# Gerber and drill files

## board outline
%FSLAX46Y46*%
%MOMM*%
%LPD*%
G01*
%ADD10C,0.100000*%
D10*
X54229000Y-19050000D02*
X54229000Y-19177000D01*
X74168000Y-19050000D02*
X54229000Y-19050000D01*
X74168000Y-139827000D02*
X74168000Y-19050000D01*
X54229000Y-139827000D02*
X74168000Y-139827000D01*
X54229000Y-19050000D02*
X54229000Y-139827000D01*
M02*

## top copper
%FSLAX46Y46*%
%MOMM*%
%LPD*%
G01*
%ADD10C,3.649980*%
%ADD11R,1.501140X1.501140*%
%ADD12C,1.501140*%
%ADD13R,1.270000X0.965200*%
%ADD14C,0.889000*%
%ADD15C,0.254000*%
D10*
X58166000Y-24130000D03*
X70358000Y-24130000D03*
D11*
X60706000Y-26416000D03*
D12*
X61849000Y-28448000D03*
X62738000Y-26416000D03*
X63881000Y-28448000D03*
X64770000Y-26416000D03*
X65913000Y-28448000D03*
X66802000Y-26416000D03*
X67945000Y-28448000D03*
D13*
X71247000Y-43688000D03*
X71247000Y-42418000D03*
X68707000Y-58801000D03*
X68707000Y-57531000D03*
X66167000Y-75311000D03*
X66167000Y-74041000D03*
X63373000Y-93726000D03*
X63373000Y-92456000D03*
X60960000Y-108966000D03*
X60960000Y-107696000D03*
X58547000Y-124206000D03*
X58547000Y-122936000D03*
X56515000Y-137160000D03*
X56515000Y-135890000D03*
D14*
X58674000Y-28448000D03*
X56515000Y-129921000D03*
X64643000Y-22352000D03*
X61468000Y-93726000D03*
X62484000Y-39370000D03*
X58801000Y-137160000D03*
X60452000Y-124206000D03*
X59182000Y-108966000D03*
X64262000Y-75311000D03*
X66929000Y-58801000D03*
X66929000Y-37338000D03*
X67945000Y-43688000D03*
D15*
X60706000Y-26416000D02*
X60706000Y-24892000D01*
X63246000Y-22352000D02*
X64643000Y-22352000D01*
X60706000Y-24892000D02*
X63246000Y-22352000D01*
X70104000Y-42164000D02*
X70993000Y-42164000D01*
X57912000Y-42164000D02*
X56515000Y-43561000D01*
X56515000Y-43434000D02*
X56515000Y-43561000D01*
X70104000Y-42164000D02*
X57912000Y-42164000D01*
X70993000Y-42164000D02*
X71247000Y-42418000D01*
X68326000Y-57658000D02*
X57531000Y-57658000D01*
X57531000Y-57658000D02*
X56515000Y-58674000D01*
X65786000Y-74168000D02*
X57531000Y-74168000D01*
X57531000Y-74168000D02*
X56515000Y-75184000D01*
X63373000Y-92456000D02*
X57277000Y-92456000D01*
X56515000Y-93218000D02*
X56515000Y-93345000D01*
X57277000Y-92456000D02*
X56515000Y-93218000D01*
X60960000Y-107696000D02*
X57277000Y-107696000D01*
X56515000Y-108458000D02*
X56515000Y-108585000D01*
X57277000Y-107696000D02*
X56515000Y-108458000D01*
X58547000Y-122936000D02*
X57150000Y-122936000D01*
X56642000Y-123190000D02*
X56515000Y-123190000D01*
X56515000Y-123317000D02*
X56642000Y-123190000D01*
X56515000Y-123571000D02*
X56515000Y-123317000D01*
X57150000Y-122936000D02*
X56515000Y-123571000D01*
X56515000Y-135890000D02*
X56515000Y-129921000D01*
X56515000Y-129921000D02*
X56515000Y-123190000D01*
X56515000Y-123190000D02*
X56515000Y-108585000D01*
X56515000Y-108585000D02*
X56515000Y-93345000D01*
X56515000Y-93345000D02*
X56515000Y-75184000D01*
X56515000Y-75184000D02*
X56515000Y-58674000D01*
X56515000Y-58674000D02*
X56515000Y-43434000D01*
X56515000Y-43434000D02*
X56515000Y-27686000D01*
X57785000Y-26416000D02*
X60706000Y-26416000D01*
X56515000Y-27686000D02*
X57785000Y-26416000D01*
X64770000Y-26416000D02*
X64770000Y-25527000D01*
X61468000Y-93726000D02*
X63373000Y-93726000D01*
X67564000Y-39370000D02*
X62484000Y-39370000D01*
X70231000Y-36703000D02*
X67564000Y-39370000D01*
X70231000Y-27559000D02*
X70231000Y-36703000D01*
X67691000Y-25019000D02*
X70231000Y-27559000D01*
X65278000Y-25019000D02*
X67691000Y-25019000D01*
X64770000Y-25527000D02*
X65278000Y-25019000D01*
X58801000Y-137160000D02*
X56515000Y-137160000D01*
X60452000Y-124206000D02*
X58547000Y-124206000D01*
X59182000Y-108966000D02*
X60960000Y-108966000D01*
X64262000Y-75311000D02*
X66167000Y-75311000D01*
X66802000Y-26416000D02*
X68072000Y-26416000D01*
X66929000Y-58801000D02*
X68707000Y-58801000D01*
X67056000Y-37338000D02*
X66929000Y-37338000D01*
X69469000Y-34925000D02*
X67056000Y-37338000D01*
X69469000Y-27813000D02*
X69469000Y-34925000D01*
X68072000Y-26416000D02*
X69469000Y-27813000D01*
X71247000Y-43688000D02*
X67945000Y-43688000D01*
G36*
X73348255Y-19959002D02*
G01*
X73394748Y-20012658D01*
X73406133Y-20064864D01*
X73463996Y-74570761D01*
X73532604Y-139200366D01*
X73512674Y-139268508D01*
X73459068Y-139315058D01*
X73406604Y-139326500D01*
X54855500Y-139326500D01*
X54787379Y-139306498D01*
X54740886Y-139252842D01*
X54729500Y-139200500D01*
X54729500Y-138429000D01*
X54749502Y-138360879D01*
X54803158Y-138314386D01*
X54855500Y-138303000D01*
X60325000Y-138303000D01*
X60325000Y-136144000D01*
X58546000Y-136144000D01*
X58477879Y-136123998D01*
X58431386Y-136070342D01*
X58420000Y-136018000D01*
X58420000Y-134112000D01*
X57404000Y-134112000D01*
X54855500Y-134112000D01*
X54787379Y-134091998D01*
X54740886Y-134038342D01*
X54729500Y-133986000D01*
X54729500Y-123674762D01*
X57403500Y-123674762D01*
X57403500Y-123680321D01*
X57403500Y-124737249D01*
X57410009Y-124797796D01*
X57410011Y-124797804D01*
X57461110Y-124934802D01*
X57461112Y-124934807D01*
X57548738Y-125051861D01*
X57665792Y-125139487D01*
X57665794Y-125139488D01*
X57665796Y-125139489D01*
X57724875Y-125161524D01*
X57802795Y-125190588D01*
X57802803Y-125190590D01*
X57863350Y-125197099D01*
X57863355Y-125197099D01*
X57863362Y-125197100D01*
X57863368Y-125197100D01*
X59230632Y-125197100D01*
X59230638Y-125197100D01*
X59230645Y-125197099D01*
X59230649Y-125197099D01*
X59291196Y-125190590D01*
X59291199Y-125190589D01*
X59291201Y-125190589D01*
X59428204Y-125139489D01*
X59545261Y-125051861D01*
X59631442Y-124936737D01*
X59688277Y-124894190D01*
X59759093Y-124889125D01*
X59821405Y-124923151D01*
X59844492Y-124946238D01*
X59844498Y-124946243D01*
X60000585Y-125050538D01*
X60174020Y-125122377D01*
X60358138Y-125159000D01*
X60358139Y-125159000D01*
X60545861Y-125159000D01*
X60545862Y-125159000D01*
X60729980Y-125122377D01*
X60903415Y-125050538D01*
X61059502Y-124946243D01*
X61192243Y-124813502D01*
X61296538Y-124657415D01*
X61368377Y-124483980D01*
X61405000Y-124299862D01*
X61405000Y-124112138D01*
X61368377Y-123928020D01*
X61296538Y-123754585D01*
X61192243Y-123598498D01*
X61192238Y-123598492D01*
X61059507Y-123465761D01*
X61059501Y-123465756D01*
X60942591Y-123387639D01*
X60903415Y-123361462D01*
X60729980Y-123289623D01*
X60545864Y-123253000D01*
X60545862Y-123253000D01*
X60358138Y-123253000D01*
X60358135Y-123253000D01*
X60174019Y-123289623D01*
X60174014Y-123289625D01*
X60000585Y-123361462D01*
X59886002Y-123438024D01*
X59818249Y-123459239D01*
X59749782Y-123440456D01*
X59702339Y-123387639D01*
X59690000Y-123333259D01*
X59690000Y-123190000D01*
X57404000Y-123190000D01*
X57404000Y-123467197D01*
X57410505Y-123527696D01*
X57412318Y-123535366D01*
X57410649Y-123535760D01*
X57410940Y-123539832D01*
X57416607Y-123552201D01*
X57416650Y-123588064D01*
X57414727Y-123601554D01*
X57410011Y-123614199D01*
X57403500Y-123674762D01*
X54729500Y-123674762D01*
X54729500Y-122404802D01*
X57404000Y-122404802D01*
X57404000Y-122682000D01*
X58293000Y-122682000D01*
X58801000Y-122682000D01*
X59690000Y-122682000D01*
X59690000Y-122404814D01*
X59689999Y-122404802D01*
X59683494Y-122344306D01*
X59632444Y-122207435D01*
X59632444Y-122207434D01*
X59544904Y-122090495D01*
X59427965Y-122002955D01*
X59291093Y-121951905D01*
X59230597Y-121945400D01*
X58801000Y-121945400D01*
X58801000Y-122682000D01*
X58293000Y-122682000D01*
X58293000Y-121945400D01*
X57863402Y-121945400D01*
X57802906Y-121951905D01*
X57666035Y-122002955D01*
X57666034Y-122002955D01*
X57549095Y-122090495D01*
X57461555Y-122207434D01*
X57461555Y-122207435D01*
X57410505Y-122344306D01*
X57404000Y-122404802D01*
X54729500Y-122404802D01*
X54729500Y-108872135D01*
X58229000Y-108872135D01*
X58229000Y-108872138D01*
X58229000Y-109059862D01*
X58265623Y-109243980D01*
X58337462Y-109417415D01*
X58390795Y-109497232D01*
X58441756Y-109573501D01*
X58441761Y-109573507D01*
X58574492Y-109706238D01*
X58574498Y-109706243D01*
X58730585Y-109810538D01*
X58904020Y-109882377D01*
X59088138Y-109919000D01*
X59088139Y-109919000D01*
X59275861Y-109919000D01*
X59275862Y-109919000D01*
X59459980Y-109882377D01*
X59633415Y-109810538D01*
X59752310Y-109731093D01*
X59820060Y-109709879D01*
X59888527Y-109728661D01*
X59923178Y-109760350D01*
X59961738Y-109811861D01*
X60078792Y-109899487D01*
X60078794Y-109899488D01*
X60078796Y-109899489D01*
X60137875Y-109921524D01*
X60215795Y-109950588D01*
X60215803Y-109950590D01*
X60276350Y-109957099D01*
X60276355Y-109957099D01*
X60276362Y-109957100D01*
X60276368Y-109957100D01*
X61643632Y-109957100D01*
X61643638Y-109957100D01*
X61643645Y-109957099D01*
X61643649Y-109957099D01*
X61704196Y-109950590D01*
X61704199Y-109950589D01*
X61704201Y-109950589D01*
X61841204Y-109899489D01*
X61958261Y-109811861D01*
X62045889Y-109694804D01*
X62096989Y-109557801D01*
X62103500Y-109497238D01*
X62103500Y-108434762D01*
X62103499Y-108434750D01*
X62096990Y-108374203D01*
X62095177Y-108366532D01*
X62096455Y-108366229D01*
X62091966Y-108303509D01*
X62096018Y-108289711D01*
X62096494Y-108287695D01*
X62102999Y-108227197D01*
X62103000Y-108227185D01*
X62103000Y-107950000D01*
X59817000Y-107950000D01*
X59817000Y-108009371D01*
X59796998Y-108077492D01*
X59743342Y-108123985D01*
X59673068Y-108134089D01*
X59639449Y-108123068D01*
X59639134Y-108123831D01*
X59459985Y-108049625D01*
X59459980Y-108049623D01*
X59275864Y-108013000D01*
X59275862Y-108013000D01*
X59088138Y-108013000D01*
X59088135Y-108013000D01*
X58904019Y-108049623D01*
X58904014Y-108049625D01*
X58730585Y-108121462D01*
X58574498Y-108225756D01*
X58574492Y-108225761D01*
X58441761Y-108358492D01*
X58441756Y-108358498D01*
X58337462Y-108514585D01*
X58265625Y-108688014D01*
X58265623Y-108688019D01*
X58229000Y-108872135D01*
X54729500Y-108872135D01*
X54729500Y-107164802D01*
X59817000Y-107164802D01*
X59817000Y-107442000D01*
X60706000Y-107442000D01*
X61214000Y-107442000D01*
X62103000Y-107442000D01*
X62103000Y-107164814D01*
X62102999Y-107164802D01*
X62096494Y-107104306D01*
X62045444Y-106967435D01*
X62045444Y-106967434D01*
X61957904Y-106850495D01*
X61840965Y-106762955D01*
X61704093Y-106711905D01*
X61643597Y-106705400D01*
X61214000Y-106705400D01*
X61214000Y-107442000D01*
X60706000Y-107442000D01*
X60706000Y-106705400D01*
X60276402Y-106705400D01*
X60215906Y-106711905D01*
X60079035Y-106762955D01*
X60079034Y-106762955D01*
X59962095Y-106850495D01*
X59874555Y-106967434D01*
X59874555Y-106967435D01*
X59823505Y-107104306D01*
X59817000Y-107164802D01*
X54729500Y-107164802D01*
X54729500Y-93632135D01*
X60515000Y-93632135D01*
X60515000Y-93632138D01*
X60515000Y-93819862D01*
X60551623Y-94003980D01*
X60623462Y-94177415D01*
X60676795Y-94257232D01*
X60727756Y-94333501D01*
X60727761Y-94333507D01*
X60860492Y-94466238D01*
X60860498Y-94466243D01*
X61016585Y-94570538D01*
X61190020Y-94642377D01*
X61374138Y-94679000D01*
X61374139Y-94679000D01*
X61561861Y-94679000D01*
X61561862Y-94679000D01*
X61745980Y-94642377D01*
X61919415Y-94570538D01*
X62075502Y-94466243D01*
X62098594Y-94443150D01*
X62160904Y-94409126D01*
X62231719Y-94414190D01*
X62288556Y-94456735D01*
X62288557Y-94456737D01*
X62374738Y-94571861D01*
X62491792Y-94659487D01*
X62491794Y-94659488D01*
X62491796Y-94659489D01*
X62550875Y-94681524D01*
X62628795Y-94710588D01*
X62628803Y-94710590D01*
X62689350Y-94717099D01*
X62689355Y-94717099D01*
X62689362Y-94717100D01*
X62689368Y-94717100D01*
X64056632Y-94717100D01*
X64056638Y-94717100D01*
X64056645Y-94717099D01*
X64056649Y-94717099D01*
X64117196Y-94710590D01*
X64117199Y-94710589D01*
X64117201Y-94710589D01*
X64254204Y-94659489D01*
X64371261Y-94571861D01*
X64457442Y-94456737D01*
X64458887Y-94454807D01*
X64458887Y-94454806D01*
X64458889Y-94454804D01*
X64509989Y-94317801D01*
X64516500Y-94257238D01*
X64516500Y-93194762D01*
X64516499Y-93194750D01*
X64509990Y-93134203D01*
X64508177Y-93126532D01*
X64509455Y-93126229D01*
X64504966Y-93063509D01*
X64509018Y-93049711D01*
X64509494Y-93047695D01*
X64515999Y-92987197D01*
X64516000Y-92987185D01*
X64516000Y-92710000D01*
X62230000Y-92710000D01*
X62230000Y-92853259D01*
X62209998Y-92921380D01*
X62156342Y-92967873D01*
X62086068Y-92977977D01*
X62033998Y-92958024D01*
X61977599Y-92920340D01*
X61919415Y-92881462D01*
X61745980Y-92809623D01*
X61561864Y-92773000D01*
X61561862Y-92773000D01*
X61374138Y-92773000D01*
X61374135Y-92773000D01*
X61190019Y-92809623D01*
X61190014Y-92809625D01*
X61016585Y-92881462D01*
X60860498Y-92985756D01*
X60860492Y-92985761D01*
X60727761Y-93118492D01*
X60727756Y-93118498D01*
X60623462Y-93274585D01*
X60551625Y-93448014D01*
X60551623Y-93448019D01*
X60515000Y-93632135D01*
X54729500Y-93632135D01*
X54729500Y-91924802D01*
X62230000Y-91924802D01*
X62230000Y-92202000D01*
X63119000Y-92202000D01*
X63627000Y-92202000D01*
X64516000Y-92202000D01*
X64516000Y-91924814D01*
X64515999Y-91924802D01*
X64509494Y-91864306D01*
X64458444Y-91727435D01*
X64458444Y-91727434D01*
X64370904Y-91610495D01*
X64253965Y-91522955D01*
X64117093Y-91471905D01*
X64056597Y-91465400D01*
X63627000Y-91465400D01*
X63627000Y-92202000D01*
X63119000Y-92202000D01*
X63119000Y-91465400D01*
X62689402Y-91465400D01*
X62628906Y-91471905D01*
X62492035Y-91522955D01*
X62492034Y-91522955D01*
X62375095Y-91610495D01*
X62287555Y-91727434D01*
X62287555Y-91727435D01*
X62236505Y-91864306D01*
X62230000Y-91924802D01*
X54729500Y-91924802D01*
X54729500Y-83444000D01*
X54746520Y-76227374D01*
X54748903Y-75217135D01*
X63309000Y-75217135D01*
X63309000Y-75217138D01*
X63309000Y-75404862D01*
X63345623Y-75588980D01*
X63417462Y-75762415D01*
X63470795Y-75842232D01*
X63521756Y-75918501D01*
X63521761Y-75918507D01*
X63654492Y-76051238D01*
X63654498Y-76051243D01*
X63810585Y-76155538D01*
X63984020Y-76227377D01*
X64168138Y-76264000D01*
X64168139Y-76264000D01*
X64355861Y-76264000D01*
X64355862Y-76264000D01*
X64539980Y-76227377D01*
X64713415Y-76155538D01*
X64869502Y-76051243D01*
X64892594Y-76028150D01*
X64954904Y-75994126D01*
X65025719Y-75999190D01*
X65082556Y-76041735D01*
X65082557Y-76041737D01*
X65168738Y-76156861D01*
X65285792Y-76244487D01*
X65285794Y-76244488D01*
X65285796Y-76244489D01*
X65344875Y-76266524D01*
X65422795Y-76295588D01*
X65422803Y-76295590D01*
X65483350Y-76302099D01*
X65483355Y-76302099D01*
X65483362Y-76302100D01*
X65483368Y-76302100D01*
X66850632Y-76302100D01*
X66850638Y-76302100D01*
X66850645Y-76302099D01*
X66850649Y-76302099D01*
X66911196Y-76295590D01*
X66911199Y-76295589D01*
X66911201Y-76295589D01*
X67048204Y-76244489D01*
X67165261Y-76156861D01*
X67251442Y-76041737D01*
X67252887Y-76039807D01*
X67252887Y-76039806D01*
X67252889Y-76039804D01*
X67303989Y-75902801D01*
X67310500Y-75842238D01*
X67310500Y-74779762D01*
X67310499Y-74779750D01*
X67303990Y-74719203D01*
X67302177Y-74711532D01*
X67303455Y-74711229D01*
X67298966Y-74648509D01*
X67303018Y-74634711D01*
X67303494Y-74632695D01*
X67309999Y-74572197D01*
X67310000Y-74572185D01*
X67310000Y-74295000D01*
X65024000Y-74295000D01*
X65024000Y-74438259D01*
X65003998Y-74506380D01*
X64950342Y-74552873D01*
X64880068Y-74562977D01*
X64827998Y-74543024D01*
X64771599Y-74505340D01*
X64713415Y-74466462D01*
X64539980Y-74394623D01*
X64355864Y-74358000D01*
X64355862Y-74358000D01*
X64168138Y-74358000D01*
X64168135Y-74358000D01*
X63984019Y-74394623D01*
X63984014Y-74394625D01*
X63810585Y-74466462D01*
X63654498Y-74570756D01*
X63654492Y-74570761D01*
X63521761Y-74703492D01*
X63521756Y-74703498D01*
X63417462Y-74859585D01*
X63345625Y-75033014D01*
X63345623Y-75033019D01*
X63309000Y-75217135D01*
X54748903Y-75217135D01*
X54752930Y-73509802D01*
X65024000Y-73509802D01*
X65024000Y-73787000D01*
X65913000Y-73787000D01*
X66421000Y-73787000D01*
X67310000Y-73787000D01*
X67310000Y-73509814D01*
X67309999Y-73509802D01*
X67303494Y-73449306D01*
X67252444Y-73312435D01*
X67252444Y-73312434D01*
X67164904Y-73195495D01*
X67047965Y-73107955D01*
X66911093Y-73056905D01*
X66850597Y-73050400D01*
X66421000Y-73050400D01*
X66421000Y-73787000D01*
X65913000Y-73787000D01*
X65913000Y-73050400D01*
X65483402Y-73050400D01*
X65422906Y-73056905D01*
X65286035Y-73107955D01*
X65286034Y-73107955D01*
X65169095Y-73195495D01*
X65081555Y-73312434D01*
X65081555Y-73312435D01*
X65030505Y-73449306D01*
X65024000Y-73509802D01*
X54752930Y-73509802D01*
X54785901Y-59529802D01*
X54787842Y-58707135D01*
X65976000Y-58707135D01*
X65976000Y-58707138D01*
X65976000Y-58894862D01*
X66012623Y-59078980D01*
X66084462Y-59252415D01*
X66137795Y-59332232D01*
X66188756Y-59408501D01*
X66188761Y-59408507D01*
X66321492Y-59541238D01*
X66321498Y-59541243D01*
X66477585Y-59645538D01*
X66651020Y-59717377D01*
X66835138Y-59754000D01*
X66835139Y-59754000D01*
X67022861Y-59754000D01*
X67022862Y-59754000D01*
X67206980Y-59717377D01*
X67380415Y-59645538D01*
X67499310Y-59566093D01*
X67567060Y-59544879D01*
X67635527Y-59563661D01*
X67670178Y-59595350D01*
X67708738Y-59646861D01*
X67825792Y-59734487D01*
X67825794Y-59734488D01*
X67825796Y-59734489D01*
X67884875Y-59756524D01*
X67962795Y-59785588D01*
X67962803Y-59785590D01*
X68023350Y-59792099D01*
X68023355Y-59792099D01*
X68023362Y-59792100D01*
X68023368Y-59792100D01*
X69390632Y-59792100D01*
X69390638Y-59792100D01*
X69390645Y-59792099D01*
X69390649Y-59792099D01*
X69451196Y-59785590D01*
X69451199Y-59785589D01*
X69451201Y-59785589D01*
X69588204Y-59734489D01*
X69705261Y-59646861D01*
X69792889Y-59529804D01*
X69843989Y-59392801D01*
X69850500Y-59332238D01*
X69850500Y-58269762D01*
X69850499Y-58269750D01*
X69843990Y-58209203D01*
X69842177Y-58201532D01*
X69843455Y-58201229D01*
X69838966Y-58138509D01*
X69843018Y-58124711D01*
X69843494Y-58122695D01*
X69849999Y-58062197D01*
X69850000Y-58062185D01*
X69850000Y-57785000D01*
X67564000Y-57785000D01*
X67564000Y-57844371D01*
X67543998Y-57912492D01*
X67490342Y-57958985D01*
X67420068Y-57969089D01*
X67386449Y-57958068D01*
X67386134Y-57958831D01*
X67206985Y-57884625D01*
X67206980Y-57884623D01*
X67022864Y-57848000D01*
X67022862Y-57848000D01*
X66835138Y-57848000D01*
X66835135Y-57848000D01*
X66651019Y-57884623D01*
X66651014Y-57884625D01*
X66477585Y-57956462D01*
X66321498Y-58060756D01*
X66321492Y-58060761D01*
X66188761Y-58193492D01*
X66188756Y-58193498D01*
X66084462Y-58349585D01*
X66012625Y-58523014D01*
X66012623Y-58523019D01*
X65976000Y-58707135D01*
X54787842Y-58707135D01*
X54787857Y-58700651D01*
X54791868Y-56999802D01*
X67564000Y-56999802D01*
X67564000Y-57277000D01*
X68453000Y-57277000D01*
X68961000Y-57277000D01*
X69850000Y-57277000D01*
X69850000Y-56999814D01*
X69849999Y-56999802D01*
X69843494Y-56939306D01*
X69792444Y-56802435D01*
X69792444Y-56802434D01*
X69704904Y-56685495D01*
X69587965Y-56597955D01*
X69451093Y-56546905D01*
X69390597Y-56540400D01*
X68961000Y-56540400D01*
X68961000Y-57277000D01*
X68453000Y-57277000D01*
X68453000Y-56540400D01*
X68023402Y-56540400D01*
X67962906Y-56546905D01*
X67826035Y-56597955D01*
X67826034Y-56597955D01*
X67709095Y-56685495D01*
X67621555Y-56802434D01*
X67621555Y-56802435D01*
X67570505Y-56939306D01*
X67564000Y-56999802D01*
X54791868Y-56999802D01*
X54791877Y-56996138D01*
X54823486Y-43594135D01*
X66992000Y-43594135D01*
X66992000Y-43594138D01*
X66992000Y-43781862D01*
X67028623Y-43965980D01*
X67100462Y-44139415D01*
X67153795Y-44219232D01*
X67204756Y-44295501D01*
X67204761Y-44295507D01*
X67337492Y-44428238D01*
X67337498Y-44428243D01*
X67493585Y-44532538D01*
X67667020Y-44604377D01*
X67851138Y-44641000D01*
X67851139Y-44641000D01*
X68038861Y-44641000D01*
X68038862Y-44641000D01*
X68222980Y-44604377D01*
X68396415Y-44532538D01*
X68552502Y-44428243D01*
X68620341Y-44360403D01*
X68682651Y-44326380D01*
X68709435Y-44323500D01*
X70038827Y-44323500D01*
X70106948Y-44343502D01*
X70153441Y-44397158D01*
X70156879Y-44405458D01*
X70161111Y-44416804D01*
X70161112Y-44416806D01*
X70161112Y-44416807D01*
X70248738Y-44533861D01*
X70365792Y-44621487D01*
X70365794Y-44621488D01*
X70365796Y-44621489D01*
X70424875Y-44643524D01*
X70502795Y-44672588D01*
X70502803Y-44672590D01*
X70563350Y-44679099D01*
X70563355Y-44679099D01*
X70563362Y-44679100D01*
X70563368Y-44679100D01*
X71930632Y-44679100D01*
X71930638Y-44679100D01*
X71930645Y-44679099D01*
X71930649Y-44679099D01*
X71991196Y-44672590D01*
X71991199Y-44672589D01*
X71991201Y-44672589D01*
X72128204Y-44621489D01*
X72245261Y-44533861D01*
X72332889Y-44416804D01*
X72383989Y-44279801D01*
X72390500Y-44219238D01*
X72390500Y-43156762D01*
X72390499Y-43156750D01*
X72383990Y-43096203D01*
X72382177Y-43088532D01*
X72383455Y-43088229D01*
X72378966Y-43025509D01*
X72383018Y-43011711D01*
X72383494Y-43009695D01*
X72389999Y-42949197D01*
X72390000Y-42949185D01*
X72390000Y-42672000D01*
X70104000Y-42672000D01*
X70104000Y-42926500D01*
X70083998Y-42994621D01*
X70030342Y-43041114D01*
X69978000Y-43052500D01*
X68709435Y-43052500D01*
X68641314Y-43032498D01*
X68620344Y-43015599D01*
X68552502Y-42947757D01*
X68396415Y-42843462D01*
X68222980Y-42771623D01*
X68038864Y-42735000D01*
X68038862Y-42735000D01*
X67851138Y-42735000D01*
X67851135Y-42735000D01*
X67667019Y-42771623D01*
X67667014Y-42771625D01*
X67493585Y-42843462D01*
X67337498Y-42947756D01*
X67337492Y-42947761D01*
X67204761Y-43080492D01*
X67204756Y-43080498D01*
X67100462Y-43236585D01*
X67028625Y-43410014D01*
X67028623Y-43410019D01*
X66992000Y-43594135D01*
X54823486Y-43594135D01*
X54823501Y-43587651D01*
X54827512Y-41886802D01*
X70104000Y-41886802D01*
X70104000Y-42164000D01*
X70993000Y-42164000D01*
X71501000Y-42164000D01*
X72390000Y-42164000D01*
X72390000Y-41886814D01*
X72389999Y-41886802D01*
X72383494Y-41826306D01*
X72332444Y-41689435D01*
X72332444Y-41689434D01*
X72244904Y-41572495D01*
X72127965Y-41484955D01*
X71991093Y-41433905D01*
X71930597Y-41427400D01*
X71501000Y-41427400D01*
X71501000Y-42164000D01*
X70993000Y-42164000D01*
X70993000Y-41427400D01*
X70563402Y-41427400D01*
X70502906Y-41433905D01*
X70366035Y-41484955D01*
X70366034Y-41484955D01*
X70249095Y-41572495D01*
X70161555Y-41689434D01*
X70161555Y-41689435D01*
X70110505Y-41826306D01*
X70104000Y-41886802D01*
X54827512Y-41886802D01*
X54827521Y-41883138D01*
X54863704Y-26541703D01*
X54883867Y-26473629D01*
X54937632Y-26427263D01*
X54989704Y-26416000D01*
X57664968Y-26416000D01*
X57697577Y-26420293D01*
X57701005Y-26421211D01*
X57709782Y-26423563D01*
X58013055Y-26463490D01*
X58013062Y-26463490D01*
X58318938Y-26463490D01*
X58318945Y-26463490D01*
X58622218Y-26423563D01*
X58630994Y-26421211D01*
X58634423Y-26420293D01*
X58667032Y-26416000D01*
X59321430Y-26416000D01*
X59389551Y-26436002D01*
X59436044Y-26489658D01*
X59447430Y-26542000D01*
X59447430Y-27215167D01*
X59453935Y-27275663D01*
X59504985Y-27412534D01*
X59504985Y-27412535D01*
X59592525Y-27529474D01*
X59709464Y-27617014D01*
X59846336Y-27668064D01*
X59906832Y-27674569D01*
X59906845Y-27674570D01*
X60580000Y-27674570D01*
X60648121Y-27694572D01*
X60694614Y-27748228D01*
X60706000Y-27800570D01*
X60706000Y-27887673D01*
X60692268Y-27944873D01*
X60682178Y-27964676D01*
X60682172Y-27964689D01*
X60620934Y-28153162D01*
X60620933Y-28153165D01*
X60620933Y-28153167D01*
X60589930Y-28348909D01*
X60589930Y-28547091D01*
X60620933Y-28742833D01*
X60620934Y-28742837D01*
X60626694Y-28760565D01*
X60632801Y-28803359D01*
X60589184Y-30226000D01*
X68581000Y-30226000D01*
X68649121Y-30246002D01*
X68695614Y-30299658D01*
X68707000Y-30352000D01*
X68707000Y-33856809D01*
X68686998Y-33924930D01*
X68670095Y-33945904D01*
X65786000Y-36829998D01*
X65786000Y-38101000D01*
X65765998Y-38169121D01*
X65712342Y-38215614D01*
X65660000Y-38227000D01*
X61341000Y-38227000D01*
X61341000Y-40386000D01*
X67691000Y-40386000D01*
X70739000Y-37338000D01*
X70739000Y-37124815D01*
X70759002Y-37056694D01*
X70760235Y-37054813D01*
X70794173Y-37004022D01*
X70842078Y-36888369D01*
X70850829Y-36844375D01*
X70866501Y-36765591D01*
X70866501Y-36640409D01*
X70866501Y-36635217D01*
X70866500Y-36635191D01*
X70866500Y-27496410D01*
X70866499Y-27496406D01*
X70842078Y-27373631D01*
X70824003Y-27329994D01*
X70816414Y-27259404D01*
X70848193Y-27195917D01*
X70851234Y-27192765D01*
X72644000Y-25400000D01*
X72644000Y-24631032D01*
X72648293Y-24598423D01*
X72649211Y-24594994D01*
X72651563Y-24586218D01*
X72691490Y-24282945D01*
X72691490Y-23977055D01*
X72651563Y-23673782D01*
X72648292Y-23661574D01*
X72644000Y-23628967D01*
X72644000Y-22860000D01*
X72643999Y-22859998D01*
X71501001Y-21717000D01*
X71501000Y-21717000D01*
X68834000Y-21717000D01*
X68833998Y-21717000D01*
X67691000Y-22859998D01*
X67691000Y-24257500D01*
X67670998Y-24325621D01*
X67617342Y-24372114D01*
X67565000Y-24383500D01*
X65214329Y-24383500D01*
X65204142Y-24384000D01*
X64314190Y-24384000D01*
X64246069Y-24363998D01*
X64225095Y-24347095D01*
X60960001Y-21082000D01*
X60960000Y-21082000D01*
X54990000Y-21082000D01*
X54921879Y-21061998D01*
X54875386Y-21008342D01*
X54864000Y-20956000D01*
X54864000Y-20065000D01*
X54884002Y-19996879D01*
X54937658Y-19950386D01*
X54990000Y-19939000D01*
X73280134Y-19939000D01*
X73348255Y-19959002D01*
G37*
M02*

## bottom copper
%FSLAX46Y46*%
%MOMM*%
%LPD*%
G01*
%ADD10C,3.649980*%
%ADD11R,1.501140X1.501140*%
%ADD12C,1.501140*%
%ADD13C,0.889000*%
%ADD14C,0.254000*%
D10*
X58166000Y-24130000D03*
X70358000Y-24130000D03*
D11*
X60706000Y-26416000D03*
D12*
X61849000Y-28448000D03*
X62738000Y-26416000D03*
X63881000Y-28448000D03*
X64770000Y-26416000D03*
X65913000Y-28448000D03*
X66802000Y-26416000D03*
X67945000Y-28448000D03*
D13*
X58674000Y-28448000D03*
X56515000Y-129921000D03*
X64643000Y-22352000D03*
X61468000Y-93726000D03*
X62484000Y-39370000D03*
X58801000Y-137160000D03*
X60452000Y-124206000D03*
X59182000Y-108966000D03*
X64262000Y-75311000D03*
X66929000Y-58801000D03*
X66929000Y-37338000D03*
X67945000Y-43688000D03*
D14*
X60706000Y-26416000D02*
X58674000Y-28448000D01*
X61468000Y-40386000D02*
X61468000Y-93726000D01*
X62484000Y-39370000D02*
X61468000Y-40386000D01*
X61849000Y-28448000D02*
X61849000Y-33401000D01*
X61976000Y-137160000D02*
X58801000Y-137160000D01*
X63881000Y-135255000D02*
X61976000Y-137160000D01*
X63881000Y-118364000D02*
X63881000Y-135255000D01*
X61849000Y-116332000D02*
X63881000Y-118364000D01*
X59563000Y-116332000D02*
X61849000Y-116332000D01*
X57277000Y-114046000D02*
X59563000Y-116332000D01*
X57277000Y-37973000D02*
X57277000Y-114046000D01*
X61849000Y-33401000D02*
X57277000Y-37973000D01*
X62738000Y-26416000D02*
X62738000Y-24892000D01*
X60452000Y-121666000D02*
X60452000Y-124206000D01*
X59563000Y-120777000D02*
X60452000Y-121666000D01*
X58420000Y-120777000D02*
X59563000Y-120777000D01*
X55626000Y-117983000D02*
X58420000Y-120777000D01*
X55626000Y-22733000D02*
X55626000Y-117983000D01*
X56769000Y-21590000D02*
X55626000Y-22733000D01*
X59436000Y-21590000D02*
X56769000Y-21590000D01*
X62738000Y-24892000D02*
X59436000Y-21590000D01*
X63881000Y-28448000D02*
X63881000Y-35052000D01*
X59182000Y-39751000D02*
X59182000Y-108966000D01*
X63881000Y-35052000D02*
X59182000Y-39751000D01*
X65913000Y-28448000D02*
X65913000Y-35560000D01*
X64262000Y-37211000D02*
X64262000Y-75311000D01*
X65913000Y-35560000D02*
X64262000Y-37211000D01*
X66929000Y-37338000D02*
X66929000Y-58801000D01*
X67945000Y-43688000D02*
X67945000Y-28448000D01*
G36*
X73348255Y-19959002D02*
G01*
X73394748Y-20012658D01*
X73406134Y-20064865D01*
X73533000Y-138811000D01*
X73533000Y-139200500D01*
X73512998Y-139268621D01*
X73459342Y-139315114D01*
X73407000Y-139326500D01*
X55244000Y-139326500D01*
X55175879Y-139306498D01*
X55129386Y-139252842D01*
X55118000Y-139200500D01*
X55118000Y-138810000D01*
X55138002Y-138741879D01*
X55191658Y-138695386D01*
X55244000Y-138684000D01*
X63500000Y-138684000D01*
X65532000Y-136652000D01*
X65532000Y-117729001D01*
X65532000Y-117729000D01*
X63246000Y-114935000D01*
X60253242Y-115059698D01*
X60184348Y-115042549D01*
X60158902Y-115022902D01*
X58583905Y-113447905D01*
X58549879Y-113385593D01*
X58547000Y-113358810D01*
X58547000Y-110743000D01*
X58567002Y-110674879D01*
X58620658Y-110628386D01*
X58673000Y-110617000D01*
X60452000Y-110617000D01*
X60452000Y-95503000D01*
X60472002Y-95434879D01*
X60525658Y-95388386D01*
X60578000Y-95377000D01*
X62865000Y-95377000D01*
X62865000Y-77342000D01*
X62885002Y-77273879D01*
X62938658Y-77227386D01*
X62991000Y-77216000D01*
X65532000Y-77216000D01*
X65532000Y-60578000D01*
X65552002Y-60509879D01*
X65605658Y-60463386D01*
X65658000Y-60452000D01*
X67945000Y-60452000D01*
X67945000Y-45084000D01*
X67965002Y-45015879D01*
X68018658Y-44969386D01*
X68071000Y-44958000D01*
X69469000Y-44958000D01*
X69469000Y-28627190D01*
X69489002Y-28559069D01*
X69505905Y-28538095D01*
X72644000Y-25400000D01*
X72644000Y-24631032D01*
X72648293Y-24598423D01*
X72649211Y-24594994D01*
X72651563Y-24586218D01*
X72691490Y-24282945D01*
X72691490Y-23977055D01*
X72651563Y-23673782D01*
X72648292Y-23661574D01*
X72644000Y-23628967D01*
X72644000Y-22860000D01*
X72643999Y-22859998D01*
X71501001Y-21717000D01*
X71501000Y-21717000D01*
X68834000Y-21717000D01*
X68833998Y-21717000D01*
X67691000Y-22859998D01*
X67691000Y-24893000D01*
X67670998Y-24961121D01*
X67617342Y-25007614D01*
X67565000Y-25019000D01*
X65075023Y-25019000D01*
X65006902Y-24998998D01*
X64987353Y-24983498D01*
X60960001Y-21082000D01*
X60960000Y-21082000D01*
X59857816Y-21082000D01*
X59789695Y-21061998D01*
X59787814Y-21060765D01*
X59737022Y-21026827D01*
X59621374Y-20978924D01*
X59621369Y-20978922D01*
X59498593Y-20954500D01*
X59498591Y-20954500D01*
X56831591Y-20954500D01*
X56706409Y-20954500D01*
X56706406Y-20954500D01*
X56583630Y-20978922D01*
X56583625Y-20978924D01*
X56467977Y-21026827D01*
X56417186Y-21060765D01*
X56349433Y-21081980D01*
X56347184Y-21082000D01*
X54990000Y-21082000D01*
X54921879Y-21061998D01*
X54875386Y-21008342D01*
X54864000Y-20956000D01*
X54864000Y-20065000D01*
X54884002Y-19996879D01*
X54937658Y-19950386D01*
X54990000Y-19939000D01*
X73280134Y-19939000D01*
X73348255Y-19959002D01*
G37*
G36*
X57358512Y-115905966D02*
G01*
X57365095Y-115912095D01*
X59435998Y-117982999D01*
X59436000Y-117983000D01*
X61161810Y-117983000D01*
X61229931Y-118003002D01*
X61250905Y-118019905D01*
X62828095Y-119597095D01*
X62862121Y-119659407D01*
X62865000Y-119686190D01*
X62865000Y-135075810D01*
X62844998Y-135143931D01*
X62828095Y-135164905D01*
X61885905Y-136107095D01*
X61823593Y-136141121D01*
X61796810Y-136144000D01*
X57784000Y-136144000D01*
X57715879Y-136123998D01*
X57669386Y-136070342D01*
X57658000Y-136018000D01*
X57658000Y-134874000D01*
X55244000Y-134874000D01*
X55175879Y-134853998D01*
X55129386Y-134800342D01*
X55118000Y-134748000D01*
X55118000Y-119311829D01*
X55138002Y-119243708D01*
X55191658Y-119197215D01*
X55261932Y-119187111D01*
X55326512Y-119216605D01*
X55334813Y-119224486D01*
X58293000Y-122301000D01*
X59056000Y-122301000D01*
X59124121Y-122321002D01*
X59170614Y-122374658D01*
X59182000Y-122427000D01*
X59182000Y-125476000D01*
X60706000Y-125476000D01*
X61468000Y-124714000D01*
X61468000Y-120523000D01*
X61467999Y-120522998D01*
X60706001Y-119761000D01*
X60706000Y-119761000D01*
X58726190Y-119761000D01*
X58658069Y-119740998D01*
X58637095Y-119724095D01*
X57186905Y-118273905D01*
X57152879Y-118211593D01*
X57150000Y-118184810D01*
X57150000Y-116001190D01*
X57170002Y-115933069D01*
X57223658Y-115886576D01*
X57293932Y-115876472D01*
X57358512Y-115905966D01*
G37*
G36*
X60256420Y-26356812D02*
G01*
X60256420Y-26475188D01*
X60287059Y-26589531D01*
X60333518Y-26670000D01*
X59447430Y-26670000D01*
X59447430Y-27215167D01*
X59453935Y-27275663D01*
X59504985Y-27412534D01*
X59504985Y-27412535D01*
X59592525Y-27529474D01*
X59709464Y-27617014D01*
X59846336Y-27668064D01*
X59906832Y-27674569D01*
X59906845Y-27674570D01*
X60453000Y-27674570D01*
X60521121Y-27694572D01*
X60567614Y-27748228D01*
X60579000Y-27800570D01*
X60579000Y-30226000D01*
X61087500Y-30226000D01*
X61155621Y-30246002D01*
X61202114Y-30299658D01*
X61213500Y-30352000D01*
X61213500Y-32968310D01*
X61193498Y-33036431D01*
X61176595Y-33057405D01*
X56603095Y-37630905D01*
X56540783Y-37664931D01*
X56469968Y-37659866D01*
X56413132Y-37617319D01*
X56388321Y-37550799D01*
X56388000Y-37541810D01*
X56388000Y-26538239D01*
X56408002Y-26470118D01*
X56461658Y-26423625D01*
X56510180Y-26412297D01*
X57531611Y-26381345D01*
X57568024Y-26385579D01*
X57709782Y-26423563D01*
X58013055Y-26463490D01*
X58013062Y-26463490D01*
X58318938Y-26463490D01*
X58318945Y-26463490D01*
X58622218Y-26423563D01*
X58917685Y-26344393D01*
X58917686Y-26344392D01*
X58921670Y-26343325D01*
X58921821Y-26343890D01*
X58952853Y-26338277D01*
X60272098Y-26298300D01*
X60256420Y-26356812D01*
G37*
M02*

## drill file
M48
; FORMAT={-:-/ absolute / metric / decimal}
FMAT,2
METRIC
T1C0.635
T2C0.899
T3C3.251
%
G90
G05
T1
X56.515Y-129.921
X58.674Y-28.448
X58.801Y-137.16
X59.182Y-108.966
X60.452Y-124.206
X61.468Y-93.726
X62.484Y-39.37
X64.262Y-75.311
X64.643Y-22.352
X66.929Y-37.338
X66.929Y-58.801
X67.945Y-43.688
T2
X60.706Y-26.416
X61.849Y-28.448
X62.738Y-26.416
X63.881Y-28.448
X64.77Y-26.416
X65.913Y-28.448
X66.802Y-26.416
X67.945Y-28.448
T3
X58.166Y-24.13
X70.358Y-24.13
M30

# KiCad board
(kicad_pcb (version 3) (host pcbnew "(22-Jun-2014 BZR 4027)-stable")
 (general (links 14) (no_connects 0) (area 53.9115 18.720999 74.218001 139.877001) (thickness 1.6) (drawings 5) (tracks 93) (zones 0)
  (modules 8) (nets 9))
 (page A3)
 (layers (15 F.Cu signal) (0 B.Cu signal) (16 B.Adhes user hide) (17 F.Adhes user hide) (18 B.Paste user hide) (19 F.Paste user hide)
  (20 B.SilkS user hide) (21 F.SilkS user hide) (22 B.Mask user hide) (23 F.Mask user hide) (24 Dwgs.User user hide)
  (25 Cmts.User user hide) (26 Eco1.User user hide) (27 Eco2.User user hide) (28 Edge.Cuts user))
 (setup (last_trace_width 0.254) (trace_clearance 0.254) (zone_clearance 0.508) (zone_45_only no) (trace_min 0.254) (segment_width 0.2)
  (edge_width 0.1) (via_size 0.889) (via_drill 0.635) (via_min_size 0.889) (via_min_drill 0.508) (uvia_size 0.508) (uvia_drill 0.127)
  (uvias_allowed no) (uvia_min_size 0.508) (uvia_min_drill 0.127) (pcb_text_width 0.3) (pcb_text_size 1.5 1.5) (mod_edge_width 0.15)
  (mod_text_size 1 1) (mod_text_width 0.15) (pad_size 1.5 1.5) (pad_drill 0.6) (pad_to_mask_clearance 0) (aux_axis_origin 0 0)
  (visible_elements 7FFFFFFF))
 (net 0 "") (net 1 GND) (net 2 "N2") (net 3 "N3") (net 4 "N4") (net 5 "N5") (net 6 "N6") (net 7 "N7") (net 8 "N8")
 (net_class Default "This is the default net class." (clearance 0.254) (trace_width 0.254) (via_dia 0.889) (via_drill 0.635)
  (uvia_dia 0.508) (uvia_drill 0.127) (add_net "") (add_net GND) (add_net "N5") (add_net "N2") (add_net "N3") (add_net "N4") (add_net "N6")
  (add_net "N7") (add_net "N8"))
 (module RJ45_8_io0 (layer F.Cu) (at 64.262 24.13 180)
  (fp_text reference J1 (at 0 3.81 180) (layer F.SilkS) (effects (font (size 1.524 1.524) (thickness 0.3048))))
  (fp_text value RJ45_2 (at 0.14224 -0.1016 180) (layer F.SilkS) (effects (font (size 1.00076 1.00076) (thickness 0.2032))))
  (pad Hole thru_hole circle (at 6.096 0 180) (size 3.64998 3.64998) (drill 3.2512) (layers *.Cu *.Mask F.SilkS))
  (pad Hole thru_hole circle (at -6.096 0 180) (size 3.64998 3.64998) (drill 3.2512) (layers *.Cu *.Mask F.SilkS))
  (pad 1 thru_hole rect (at 3.556 -2.286) (size 1.50114 1.50114) (drill 0.89916) (layers *.Cu *.Mask F.SilkS) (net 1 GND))
  (pad 2 thru_hole circle (at 2.413 -4.318) (size 1.50114 1.50114) (drill 0.89916) (layers *.Cu *.Mask F.SilkS) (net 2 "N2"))
  (pad 3 thru_hole circle (at 1.524 -2.286) (size 1.50114 1.50114) (drill 0.89916) (layers *.Cu *.Mask F.SilkS) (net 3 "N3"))
  (pad 4 thru_hole circle (at 0.381 -4.318) (size 1.50114 1.50114) (drill 0.89916) (layers *.Cu *.Mask F.SilkS) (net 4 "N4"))
  (pad 5 thru_hole circle (at -0.508 -2.286) (size 1.50114 1.50114) (drill 0.89916) (layers *.Cu *.Mask F.SilkS) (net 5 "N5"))
  (pad 6 thru_hole circle (at -1.651 -4.318) (size 1.50114 1.50114) (drill 0.89916) (layers *.Cu *.Mask F.SilkS) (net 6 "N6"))
  (pad 7 thru_hole circle (at -2.54 -2.286) (size 1.50114 1.50114) (drill 0.89916) (layers *.Cu *.Mask F.SilkS) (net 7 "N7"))
  (pad 8 thru_hole circle (at -3.683 -4.318) (size 1.50114 1.50114) (drill 0.89916) (layers *.Cu *.Mask F.SilkS) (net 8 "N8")))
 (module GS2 (layer F.Cu) (at 71.247 43.053 180)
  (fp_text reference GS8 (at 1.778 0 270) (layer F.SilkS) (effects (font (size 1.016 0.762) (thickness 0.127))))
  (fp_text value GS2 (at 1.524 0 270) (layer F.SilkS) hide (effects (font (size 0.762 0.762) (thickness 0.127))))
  (pad 1 smd rect (at 0 -0.635 180) (size 1.27 0.9652) (layers F.Cu F.Paste F.Mask) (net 8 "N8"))
  (pad 2 smd rect (at 0 0.635 180) (size 1.27 0.9652) (layers F.Cu F.Paste F.Mask) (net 1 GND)))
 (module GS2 (layer F.Cu) (at 68.707 58.166 180)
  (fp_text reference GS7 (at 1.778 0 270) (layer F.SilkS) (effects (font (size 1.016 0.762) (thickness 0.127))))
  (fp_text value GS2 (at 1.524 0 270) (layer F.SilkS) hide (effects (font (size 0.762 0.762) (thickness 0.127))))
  (pad 1 smd rect (at 0 -0.635 180) (size 1.27 0.9652) (layers F.Cu F.Paste F.Mask) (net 7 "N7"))
  (pad 2 smd rect (at 0 0.635 180) (size 1.27 0.9652) (layers F.Cu F.Paste F.Mask) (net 1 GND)))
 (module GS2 (layer F.Cu) (at 66.167 74.676 180)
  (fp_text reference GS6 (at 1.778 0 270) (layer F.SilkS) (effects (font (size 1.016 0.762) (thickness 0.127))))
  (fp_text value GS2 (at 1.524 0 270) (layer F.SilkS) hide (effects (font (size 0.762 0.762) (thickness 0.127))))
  (pad 1 smd rect (at 0 -0.635 180) (size 1.27 0.9652) (layers F.Cu F.Paste F.Mask) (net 6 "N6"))
  (pad 2 smd rect (at 0 0.635 180) (size 1.27 0.9652) (layers F.Cu F.Paste F.Mask) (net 1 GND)))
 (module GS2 (layer F.Cu) (at 63.373 93.091 180)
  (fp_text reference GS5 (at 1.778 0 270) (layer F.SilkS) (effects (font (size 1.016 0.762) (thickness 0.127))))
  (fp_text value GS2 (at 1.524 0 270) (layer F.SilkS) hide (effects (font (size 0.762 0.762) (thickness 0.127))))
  (pad 1 smd rect (at 0 -0.635 180) (size 1.27 0.9652) (layers F.Cu F.Paste F.Mask) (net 5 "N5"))
  (pad 2 smd rect (at 0 0.635 180) (size 1.27 0.9652) (layers F.Cu F.Paste F.Mask) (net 1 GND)))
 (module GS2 (layer F.Cu) (at 60.96 108.331 180)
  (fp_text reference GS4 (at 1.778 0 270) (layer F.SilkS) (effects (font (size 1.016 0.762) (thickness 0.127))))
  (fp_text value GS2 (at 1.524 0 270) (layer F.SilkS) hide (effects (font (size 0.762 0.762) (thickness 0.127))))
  (pad 1 smd rect (at 0 -0.635 180) (size 1.27 0.9652) (layers F.Cu F.Paste F.Mask) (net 4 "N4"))
  (pad 2 smd rect (at 0 0.635 180) (size 1.27 0.9652) (layers F.Cu F.Paste F.Mask) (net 1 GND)))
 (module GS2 (layer F.Cu) (at 58.547 123.571 180)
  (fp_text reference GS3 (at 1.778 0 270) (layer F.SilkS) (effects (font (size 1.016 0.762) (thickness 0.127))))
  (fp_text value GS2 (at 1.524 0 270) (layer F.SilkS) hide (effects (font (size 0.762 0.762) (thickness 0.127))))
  (pad 1 smd rect (at 0 -0.635 180) (size 1.27 0.9652) (layers F.Cu F.Paste F.Mask) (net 3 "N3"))
  (pad 2 smd rect (at 0 0.635 180) (size 1.27 0.9652) (layers F.Cu F.Paste F.Mask) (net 1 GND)))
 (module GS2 (layer F.Cu) (at 56.515 136.525 180)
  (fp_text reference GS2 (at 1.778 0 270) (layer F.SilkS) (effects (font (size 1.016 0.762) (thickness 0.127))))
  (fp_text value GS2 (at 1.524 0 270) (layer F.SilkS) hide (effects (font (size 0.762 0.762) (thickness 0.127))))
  (pad 1 smd rect (at 0 -0.635 180) (size 1.27 0.9652) (layers F.Cu F.Paste F.Mask) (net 2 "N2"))
  (pad 2 smd rect (at 0 0.635 180) (size 1.27 0.9652) (layers F.Cu F.Paste F.Mask) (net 1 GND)))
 (gr_line (start 54.229 19.05) (end 54.229 19.177) (angle 90) (layer Edge.Cuts) (width 0.1))
 (gr_line (start 74.168 19.05) (end 54.229 19.05) (angle 90) (layer Edge.Cuts) (width 0.1))
 (gr_line (start 74.168 139.827) (end 74.168 19.05) (angle 90) (layer Edge.Cuts) (width 0.1))
 (gr_line (start 54.229 139.827) (end 74.168 139.827) (angle 90) (layer Edge.Cuts) (width 0.1))
 (gr_line (start 54.229 19.05) (end 54.229 139.827) (angle 90) (layer Edge.Cuts) (width 0.1))
 (segment (start 60.706 26.416) (end 58.674 28.448) (width 0.254) (layer B.Cu) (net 1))
 (via (at 58.674 28.448) (size 0.889) (layers F.Cu B.Cu) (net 1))
 (via (at 56.515 129.921) (size 0.889) (layers F.Cu B.Cu) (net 1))
 (segment (start 60.706 26.416) (end 60.706 24.892) (width 0.254) (layer F.Cu) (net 1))
 (via (at 64.643 22.352) (size 0.889) (layers F.Cu B.Cu) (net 1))
 (segment (start 63.246 22.352) (end 64.643 22.352) (width 0.254) (layer F.Cu) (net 1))
 (segment (start 60.706 24.892) (end 63.246 22.352) (width 0.254) (layer F.Cu) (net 1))
 (segment (start 70.104 42.164) (end 70.993 42.164) (width 0.254) (layer F.Cu) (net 1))
 (segment (start 57.912 42.164) (end 56.515 43.561) (width 0.254) (layer F.Cu) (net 1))
 (segment (start 56.515 43.434) (end 56.515 43.561) (width 0.254) (layer F.Cu) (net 1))
 (segment (start 70.104 42.164) (end 57.912 42.164) (width 0.254) (layer F.Cu) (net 1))
 (segment (start 70.993 42.164) (end 71.247 42.418) (width 0.254) (layer F.Cu) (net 1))
 (segment (start 68.326 57.658) (end 57.531 57.658) (width 0.254) (layer F.Cu) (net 1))
 (segment (start 57.531 57.658) (end 56.515 58.674) (width 0.254) (layer F.Cu) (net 1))
 (segment (start 65.786 74.168) (end 57.531 74.168) (width 0.254) (layer F.Cu) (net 1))
 (segment (start 57.531 74.168) (end 56.515 75.184) (width 0.254) (layer F.Cu) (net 1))
 (segment (start 63.373 92.456) (end 57.277 92.456) (width 0.254) (layer F.Cu) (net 1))
 (segment (start 56.515 93.218) (end 56.515 93.345) (width 0.254) (layer F.Cu) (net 1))
 (segment (start 57.277 92.456) (end 56.515 93.218) (width 0.254) (layer F.Cu) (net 1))
 (segment (start 60.96 107.696) (end 57.277 107.696) (width 0.254) (layer F.Cu) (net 1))
 (segment (start 56.515 108.458) (end 56.515 108.585) (width 0.254) (layer F.Cu) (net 1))
 (segment (start 57.277 107.696) (end 56.515 108.458) (width 0.254) (layer F.Cu) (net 1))
 (segment (start 58.547 122.936) (end 57.15 122.936) (width 0.254) (layer F.Cu) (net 1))
 (segment (start 56.642 123.19) (end 56.515 123.19) (width 0.254) (layer F.Cu) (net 1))
 (segment (start 56.515 123.317) (end 56.642 123.19) (width 0.254) (layer F.Cu) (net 1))
 (segment (start 56.515 123.571) (end 56.515 123.317) (width 0.254) (layer F.Cu) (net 1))
 (segment (start 57.15 122.936) (end 56.515 123.571) (width 0.254) (layer F.Cu) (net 1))
 (segment (start 56.515 135.89) (end 56.515 129.921) (width 0.254) (layer F.Cu) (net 1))
 (segment (start 56.515 129.921) (end 56.515 123.19) (width 0.254) (layer F.Cu) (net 1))
 (segment (start 56.515 123.19) (end 56.515 108.585) (width 0.254) (layer F.Cu) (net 1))
 (segment (start 56.515 108.585) (end 56.515 93.345) (width 0.254) (layer F.Cu) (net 1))
 (segment (start 56.515 93.345) (end 56.515 75.184) (width 0.254) (layer F.Cu) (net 1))
 (segment (start 56.515 75.184) (end 56.515 58.674) (width 0.254) (layer F.Cu) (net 1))
 (segment (start 56.515 58.674) (end 56.515 43.434) (width 0.254) (layer F.Cu) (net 1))
 (segment (start 56.515 43.434) (end 56.515 27.686) (width 0.254) (layer F.Cu) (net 1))
 (segment (start 57.785 26.416) (end 60.706 26.416) (width 0.254) (layer F.Cu) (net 1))
 (segment (start 56.515 27.686) (end 57.785 26.416) (width 0.254) (layer F.Cu) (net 1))
 (segment (start 64.77 26.416) (end 64.77 25.527) (width 0.254) (layer F.Cu) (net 5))
 (segment (start 61.468 93.726) (end 63.373 93.726) (width 0.254) (layer F.Cu) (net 5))
 (via (at 61.468 93.726) (size 0.889) (layers F.Cu B.Cu) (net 5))
 (segment (start 61.468 40.386) (end 61.468 93.726) (width 0.254) (layer B.Cu) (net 5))
 (segment (start 62.484 39.37) (end 61.468 40.386) (width 0.254) (layer B.Cu) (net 5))
 (via (at 62.484 39.37) (size 0.889) (layers F.Cu B.Cu) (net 5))
 (segment (start 67.564 39.37) (end 62.484 39.37) (width 0.254) (layer F.Cu) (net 5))
 (segment (start 70.231 36.703) (end 67.564 39.37) (width 0.254) (layer F.Cu) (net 5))
 (segment (start 70.231 27.559) (end 70.231 36.703) (width 0.254) (layer F.Cu) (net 5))
 (segment (start 67.691 25.019) (end 70.231 27.559) (width 0.254) (layer F.Cu) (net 5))
 (segment (start 65.278 25.019) (end 67.691 25.019) (width 0.254) (layer F.Cu) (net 5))
 (segment (start 64.77 25.527) (end 65.278 25.019) (width 0.254) (layer F.Cu) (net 5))
 (segment (start 61.849 28.448) (end 61.849 33.401) (width 0.254) (layer B.Cu) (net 2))
 (segment (start 58.801 137.16) (end 56.515 137.16) (width 0.254) (layer F.Cu) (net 2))
 (via (at 58.801 137.16) (size 0.889) (layers F.Cu B.Cu) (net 2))
 (segment (start 61.976 137.16) (end 58.801 137.16) (width 0.254) (layer B.Cu) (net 2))
 (segment (start 63.881 135.255) (end 61.976 137.16) (width 0.254) (layer B.Cu) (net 2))
 (segment (start 63.881 118.364) (end 63.881 135.255) (width 0.254) (layer B.Cu) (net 2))
 (segment (start 61.849 116.332) (end 63.881 118.364) (width 0.254) (layer B.Cu) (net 2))
 (segment (start 59.563 116.332) (end 61.849 116.332) (width 0.254) (layer B.Cu) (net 2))
 (segment (start 57.277 114.046) (end 59.563 116.332) (width 0.254) (layer B.Cu) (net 2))
 (segment (start 57.277 37.973) (end 57.277 114.046) (width 0.254) (layer B.Cu) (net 2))
 (segment (start 61.849 33.401) (end 57.277 37.973) (width 0.254) (layer B.Cu) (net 2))
 (segment (start 62.738 26.416) (end 62.738 24.892) (width 0.254) (layer B.Cu) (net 3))
 (segment (start 60.452 124.206) (end 58.547 124.206) (width 0.254) (layer F.Cu) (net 3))
 (via (at 60.452 124.206) (size 0.889) (layers F.Cu B.Cu) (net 3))
 (segment (start 60.452 121.666) (end 60.452 124.206) (width 0.254) (layer B.Cu) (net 3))
 (segment (start 59.563 120.777) (end 60.452 121.666) (width 0.254) (layer B.Cu) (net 3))
 (segment (start 58.42 120.777) (end 59.563 120.777) (width 0.254) (layer B.Cu) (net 3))
 (segment (start 55.626 117.983) (end 58.42 120.777) (width 0.254) (layer B.Cu) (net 3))
 (segment (start 55.626 22.733) (end 55.626 117.983) (width 0.254) (layer B.Cu) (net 3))
 (segment (start 56.769 21.59) (end 55.626 22.733) (width 0.254) (layer B.Cu) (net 3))
 (segment (start 59.436 21.59) (end 56.769 21.59) (width 0.254) (layer B.Cu) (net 3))
 (segment (start 62.738 24.892) (end 59.436 21.59) (width 0.254) (layer B.Cu) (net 3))
 (segment (start 63.881 28.448) (end 63.881 35.052) (width 0.254) (layer B.Cu) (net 4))
 (segment (start 59.182 108.966) (end 60.96 108.966) (width 0.254) (layer F.Cu) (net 4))
 (via (at 59.182 108.966) (size 0.889) (layers F.Cu B.Cu) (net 4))
 (segment (start 59.182 39.751) (end 59.182 108.966) (width 0.254) (layer B.Cu) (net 4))
 (segment (start 63.881 35.052) (end 59.182 39.751) (width 0.254) (layer B.Cu) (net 4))
 (segment (start 65.913 28.448) (end 65.913 35.56) (width 0.254) (layer B.Cu) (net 6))
 (segment (start 64.262 75.311) (end 66.167 75.311) (width 0.254) (layer F.Cu) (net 6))
 (via (at 64.262 75.311) (size 0.889) (layers F.Cu B.Cu) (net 6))
 (segment (start 64.262 37.211) (end 64.262 75.311) (width 0.254) (layer B.Cu) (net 6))
 (segment (start 65.913 35.56) (end 64.262 37.211) (width 0.254) (layer B.Cu) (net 6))
 (segment (start 66.802 26.416) (end 68.072 26.416) (width 0.254) (layer F.Cu) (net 7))
 (segment (start 66.929 58.801) (end 68.707 58.801) (width 0.254) (layer F.Cu) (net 7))
 (via (at 66.929 58.801) (size 0.889) (layers F.Cu B.Cu) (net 7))
 (segment (start 66.929 37.338) (end 66.929 58.801) (width 0.254) (layer B.Cu) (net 7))
 (via (at 66.929 37.338) (size 0.889) (layers F.Cu B.Cu) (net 7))
 (segment (start 67.056 37.338) (end 66.929 37.338) (width 0.254) (layer F.Cu) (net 7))
 (segment (start 69.469 34.925) (end 67.056 37.338) (width 0.254) (layer F.Cu) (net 7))
 (segment (start 69.469 27.813) (end 69.469 34.925) (width 0.254) (layer F.Cu) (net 7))
 (segment (start 68.072 26.416) (end 69.469 27.813) (width 0.254) (layer F.Cu) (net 7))
 (segment (start 71.247 43.688) (end 67.945 43.688) (width 0.254) (layer F.Cu) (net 8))
 (via (at 67.945 43.688) (size 0.889) (layers F.Cu B.Cu) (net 8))
 (segment (start 67.945 43.688) (end 67.945 28.448) (width 0.254) (layer B.Cu) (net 8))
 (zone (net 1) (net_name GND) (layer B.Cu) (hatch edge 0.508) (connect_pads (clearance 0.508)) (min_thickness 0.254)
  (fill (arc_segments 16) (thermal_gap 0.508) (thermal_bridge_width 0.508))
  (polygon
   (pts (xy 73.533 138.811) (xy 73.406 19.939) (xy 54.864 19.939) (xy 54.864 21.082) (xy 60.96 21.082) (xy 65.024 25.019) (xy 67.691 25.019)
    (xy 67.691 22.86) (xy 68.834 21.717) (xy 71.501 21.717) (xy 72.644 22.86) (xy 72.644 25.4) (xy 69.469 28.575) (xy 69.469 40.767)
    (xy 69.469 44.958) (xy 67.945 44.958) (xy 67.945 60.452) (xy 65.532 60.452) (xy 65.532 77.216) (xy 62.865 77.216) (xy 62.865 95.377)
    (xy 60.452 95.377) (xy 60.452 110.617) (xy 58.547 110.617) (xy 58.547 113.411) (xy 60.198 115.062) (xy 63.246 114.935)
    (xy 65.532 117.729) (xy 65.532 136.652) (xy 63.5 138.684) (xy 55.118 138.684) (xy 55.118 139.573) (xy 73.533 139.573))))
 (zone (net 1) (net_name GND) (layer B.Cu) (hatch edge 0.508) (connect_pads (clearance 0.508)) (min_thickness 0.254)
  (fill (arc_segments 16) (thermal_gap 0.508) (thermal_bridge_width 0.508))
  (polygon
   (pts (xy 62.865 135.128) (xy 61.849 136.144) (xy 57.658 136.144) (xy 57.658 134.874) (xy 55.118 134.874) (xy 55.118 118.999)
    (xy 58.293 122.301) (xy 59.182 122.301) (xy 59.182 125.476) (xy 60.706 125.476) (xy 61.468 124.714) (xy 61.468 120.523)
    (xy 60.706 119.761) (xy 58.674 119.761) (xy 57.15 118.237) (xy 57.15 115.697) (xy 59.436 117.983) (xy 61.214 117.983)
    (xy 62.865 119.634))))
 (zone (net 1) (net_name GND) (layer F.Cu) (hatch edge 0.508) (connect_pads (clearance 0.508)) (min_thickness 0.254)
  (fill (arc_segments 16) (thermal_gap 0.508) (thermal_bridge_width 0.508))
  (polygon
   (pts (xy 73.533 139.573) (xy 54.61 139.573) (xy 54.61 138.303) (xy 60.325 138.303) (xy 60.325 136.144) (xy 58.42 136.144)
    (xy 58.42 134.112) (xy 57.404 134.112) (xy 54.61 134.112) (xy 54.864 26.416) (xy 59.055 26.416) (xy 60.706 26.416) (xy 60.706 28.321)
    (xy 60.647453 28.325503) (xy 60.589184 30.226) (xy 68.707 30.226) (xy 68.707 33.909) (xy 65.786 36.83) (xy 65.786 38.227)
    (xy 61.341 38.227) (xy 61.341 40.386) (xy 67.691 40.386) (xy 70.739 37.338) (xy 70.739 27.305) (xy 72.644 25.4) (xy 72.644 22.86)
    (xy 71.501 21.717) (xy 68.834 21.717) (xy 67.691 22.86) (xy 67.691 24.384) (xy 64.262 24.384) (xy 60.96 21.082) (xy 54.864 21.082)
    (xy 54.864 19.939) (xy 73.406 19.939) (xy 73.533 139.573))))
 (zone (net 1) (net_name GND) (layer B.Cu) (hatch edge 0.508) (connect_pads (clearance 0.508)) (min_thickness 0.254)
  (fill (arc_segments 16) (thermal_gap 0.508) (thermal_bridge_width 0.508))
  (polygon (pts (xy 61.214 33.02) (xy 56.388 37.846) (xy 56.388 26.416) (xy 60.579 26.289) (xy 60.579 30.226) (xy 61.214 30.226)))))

